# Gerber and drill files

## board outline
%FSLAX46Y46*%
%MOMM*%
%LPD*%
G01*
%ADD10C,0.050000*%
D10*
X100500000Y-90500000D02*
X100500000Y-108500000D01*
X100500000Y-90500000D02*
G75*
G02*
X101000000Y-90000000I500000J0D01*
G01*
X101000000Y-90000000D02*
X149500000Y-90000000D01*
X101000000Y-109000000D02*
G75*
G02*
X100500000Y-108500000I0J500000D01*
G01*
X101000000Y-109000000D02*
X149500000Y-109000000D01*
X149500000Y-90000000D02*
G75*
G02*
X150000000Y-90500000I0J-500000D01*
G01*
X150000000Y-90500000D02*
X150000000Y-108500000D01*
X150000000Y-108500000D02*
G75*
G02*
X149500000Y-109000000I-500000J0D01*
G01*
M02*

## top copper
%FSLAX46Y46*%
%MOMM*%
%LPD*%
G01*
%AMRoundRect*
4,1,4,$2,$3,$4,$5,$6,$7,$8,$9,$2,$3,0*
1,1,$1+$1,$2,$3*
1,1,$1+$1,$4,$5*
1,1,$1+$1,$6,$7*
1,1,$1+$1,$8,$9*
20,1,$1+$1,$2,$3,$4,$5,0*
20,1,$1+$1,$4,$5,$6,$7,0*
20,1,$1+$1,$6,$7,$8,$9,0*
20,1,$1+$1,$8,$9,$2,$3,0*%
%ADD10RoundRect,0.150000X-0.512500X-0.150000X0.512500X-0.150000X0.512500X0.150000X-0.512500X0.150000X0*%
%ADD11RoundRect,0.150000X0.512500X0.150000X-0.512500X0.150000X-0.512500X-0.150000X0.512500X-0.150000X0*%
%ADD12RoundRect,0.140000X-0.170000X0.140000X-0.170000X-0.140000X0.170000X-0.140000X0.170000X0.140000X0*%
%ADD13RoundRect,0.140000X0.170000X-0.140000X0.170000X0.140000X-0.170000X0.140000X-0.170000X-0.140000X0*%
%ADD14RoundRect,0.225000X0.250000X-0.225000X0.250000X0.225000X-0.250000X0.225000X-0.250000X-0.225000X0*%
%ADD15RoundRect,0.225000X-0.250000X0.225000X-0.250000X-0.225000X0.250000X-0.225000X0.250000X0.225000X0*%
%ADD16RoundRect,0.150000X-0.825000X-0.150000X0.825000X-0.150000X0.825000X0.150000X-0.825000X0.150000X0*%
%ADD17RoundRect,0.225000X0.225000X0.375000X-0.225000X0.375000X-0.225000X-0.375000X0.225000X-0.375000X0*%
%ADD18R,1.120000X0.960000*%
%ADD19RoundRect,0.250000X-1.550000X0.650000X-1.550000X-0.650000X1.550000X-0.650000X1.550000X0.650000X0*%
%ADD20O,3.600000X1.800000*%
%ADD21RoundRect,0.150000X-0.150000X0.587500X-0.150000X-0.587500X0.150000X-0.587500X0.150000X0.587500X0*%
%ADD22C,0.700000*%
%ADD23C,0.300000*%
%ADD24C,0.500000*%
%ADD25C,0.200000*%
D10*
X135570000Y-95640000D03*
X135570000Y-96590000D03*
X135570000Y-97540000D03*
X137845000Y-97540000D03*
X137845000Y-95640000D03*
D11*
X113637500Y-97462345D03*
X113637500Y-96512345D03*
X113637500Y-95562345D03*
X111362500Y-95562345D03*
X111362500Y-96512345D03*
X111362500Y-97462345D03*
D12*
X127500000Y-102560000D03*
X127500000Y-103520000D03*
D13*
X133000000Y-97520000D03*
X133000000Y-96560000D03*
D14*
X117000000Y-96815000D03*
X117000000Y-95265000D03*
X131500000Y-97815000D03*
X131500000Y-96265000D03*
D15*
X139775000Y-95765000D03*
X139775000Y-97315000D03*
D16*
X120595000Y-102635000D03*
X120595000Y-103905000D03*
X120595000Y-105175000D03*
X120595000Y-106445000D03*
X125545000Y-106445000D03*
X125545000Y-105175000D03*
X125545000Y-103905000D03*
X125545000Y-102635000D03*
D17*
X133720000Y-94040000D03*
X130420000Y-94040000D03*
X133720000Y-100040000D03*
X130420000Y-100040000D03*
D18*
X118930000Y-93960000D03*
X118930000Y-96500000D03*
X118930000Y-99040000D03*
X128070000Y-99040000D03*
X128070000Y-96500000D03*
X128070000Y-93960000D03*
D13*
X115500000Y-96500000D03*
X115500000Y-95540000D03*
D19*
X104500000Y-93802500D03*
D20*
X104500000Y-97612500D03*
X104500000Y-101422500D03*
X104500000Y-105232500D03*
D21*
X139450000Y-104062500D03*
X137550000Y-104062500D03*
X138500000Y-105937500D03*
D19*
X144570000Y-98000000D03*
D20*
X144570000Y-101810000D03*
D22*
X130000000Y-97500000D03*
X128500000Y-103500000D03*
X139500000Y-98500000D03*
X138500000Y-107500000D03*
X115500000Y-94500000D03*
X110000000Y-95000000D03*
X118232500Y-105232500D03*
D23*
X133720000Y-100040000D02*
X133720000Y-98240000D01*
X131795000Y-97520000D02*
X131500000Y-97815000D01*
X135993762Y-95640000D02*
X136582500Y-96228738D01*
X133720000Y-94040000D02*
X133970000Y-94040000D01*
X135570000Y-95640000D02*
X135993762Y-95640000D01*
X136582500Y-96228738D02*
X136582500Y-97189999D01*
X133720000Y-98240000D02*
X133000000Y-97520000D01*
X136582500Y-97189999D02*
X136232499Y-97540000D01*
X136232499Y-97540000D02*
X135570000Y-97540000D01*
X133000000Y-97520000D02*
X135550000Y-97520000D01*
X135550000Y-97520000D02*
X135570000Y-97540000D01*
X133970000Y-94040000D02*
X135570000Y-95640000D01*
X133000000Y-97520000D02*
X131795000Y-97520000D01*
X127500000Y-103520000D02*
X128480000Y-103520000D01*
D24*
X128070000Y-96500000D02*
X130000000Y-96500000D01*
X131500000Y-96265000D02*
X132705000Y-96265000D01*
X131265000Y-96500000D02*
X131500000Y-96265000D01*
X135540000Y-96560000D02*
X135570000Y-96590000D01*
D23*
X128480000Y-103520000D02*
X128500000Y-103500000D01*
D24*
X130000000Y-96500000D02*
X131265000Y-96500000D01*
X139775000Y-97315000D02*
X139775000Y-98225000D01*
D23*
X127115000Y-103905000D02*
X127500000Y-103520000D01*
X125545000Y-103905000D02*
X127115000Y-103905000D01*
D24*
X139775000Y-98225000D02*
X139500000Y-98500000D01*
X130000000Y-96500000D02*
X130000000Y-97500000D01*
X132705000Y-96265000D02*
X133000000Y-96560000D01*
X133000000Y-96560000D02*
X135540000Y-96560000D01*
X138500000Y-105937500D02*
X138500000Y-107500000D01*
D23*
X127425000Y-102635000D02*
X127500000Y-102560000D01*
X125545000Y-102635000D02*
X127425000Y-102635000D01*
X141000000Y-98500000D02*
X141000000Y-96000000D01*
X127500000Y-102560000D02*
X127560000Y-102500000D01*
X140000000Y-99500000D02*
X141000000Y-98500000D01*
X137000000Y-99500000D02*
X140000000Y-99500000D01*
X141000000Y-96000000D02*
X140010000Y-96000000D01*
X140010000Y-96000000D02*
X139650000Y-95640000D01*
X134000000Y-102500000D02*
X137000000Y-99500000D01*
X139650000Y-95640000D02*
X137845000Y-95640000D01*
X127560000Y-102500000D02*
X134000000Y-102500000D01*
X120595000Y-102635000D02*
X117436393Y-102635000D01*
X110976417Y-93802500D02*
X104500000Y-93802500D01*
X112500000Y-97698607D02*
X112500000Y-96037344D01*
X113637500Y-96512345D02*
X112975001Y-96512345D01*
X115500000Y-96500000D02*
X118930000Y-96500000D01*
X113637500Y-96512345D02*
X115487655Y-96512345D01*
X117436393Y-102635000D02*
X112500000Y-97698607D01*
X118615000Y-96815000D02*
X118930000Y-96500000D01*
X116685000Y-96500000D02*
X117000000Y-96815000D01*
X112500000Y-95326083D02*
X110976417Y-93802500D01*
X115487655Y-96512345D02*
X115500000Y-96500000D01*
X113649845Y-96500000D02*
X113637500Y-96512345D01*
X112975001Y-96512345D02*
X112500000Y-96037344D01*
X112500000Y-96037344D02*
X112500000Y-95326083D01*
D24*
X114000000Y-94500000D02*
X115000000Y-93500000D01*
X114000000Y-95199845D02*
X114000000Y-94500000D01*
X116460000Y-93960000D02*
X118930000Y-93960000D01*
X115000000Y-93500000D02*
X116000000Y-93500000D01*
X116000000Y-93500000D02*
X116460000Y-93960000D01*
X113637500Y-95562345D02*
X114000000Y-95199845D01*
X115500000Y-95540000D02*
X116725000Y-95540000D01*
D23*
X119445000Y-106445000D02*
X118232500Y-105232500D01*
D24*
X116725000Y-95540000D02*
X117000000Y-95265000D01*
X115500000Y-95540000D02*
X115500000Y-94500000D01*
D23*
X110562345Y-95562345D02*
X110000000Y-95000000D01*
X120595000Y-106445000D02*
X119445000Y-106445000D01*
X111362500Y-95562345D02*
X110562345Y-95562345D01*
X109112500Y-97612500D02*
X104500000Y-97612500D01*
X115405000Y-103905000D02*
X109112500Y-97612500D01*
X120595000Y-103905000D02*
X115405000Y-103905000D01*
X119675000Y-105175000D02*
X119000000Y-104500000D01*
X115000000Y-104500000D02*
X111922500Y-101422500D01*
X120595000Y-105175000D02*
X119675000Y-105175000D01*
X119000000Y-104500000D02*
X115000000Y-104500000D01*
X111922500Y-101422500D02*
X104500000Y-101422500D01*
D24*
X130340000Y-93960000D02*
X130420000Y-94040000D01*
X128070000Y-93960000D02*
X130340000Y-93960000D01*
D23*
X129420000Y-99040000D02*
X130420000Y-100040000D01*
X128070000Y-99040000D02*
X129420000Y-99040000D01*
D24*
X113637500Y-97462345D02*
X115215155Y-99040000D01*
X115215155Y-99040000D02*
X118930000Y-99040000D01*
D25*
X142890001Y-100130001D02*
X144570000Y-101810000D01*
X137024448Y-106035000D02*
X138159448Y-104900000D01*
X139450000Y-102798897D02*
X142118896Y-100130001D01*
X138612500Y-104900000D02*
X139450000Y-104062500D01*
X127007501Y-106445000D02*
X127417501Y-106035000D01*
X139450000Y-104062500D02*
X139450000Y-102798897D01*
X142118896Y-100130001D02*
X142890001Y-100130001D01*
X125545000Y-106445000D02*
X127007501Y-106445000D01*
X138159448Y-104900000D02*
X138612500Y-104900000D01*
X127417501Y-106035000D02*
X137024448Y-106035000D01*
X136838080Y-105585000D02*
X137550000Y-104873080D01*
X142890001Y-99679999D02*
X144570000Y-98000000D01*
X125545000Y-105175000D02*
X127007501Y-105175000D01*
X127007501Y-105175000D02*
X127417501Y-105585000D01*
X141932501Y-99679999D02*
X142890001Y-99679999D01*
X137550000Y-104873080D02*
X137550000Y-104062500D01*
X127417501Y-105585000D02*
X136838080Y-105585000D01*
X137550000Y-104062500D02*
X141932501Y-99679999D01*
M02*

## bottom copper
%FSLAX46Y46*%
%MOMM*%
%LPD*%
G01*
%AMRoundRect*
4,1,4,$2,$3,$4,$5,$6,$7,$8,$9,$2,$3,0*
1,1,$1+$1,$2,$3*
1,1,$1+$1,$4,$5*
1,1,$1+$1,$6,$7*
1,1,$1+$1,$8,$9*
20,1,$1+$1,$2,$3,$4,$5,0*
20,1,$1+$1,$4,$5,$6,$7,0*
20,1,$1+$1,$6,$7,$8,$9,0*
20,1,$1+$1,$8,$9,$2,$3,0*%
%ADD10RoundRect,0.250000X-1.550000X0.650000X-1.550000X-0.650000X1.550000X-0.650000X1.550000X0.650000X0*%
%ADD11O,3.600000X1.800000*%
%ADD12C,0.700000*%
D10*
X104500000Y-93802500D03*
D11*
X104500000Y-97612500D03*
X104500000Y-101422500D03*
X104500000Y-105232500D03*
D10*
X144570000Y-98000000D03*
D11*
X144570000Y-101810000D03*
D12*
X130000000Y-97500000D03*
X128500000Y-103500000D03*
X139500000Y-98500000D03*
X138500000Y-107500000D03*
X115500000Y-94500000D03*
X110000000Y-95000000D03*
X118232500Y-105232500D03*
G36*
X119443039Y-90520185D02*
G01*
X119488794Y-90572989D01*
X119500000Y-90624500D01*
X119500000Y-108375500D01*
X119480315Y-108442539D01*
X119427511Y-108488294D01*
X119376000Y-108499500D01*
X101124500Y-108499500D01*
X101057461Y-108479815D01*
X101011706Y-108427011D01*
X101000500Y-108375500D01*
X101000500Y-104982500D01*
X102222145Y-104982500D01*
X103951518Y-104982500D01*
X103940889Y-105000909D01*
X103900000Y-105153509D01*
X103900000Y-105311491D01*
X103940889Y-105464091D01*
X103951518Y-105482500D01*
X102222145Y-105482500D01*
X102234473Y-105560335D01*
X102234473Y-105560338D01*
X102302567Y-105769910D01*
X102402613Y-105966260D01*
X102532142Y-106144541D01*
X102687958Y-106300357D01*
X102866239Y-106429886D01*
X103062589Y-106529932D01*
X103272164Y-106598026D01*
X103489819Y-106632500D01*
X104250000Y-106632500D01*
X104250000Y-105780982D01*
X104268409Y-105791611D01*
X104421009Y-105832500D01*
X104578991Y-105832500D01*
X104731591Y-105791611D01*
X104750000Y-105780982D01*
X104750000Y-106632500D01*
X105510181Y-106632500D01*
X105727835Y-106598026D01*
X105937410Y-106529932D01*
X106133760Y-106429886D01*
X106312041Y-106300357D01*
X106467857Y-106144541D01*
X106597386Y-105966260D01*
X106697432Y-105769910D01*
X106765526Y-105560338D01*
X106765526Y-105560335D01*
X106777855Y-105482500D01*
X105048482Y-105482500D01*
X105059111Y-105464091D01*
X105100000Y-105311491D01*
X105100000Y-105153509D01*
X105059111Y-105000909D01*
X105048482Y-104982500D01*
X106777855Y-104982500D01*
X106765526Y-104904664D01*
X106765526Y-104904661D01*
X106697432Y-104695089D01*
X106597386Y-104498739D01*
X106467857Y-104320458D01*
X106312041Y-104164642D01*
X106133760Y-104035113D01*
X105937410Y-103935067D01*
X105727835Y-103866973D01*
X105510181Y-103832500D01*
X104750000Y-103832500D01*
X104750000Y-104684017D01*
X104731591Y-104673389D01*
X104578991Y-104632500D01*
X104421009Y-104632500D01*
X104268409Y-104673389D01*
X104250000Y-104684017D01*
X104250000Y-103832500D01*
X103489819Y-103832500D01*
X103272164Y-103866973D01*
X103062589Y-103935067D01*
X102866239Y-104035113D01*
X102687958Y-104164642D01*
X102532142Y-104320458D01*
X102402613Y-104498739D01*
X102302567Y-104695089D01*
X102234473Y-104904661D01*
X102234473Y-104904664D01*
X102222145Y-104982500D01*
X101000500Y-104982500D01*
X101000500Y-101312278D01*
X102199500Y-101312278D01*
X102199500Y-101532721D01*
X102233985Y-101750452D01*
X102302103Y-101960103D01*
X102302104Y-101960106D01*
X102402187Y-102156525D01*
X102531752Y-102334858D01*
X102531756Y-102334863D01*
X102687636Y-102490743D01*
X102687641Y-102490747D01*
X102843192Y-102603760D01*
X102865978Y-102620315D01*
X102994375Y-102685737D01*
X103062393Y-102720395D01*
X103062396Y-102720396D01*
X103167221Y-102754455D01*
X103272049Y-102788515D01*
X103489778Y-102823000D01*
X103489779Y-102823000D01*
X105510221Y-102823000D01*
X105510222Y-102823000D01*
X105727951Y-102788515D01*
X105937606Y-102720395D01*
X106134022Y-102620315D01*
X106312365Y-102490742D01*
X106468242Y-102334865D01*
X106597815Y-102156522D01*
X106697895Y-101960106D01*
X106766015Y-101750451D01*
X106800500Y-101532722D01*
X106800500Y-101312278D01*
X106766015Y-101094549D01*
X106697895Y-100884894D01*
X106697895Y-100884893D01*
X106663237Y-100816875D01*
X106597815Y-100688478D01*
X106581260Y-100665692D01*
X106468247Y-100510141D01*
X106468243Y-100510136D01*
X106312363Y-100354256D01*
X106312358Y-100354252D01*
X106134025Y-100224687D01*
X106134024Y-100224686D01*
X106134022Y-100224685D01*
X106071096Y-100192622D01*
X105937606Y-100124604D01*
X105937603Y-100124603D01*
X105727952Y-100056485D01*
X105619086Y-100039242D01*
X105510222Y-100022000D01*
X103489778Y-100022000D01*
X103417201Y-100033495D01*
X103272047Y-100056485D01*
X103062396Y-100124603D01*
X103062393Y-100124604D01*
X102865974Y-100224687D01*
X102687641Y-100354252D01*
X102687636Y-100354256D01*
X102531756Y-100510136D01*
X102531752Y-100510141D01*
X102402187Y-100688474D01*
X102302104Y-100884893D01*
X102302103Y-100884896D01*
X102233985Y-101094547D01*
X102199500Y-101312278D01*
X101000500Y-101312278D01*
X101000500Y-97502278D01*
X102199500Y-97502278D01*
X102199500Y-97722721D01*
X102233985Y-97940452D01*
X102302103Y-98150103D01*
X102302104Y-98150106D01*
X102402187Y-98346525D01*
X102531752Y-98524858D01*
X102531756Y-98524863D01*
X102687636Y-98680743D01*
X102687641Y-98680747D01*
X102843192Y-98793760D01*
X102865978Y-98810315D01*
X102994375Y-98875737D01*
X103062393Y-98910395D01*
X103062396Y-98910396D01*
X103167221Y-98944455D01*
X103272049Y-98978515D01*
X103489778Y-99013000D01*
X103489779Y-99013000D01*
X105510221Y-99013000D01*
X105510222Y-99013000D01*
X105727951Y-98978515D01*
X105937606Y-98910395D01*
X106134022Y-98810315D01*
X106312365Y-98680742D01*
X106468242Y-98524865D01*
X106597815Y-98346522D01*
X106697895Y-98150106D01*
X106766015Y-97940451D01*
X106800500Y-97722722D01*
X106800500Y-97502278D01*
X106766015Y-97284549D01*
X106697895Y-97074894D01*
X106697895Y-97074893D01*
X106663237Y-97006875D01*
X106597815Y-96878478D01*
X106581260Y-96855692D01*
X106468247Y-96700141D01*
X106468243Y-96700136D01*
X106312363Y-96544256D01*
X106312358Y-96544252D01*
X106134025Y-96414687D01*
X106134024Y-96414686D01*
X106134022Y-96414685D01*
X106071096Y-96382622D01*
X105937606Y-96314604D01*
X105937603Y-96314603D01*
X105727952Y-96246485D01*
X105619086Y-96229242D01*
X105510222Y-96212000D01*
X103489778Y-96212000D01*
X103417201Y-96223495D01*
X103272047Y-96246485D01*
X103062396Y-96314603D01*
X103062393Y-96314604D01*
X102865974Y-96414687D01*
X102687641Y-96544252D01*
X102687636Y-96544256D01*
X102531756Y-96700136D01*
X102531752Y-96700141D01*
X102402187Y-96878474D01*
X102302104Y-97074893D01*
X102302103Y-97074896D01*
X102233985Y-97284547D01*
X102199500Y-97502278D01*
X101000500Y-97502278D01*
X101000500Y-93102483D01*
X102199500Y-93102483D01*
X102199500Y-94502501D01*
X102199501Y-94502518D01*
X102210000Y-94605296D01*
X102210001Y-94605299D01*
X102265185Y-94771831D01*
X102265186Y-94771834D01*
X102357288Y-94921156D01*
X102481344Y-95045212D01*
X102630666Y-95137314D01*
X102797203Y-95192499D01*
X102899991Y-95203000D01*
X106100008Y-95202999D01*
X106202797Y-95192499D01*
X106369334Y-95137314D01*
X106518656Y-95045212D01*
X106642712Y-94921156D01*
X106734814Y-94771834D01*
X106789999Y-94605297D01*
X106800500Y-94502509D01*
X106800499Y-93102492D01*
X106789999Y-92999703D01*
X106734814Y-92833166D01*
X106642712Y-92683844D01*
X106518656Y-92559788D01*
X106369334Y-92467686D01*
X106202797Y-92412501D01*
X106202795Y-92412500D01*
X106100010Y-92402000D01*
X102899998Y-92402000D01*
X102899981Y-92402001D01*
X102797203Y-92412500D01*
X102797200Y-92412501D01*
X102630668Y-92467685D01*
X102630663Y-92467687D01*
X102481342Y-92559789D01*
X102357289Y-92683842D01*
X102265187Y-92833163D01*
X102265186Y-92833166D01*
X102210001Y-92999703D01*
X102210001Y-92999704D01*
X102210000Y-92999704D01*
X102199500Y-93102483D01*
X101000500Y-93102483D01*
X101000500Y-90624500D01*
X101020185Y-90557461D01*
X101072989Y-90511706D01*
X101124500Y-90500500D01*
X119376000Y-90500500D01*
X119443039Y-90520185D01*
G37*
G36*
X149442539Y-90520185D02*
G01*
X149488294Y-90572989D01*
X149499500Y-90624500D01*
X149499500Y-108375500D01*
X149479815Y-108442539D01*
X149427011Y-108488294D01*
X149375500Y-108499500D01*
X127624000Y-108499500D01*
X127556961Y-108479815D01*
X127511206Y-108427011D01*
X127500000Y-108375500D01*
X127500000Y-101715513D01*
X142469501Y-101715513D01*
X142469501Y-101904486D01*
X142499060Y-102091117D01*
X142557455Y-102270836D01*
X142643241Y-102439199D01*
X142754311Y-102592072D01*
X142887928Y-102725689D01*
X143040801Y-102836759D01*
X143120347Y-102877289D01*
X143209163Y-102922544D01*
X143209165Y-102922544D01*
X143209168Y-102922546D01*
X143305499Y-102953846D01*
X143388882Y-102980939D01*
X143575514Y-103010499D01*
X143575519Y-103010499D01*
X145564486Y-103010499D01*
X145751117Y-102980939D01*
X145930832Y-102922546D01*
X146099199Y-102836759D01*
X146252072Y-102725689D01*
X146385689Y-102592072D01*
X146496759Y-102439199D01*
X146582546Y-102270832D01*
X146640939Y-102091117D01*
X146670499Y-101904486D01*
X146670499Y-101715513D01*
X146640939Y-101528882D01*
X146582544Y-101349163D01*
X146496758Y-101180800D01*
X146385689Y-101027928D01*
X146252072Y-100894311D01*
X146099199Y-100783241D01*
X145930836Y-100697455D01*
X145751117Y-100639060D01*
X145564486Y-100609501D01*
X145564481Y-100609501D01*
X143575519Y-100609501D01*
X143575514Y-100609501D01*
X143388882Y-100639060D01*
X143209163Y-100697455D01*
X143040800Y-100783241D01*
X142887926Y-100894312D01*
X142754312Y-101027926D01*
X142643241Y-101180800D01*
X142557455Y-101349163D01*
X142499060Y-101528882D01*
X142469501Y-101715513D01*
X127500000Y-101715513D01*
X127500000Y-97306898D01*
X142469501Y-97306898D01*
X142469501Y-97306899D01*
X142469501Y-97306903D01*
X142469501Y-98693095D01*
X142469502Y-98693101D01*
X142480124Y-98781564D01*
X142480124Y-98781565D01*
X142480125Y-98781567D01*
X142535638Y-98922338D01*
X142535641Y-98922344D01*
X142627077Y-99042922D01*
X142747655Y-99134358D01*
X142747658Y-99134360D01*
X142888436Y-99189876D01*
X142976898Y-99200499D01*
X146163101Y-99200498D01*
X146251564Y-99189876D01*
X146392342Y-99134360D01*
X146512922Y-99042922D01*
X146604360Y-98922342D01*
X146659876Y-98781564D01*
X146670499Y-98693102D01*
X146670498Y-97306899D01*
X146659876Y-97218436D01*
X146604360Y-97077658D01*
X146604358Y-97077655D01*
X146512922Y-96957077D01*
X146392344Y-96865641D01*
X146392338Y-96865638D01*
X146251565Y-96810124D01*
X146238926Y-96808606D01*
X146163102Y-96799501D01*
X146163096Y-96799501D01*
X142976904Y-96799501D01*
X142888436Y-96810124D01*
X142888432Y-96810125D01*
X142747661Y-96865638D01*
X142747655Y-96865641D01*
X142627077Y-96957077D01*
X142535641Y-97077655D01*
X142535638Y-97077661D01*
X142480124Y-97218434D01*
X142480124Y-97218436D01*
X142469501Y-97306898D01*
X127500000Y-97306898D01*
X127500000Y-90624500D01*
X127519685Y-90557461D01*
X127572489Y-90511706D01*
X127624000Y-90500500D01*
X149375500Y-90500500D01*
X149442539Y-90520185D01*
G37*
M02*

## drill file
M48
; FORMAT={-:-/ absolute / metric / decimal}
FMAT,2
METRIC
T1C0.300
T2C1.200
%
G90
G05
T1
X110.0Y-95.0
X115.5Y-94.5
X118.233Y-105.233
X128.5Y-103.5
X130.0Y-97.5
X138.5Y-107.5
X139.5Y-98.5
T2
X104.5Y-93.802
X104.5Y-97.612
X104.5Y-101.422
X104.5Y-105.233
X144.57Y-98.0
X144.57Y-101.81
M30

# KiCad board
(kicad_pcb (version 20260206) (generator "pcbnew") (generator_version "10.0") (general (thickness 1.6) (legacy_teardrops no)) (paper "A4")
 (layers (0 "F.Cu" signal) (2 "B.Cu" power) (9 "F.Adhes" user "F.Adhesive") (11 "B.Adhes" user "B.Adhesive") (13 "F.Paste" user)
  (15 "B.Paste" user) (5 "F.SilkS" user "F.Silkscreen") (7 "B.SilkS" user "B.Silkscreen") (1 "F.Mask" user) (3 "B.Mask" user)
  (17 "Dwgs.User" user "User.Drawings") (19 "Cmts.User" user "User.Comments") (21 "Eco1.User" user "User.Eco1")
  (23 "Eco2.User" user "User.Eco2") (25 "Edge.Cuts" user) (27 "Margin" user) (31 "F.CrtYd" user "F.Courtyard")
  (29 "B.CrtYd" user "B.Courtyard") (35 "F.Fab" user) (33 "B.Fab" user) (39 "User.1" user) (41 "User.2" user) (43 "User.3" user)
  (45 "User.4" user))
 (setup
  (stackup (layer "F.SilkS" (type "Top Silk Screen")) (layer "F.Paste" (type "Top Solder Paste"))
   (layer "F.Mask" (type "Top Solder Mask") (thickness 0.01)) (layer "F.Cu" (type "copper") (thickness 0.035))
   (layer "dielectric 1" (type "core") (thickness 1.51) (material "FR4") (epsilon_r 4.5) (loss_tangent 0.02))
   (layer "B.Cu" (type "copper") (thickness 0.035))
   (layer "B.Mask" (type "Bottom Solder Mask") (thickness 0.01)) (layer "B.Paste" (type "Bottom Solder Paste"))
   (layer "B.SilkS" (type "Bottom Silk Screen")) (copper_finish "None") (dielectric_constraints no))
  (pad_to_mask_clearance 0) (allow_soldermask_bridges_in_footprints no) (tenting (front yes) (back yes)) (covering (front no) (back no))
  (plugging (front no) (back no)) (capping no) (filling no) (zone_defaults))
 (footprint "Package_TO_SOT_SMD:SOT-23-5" (layer "F.Cu") (at 136.7075 96.59)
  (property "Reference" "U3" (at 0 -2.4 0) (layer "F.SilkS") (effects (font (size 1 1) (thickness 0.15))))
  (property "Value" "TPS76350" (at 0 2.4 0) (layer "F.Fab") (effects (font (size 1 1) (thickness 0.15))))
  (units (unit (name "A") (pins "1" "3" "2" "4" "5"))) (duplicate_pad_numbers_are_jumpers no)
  (pad "1" smd roundrect (at -1.1375 -0.95) (size 1.325 0.6) (layers "F.Cu" "F.Mask" "F.Paste") (roundrect_rratio 0.25) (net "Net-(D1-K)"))
  (pad "2" smd roundrect (at -1.1375 0) (size 1.325 0.6) (layers "F.Cu" "F.Mask" "F.Paste") (roundrect_rratio 0.25) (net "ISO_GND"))
  (pad "3" smd roundrect (at -1.1375 0.95) (size 1.325 0.6) (layers "F.Cu" "F.Mask" "F.Paste") (roundrect_rratio 0.25) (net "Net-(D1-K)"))
  (pad "4" smd roundrect (at 1.1375 0.95) (size 1.325 0.6) (layers "F.Cu" "F.Mask" "F.Paste") (roundrect_rratio 0.25)
   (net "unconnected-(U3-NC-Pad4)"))
  (pad "5" smd roundrect (at 1.1375 -0.95) (size 1.325 0.6) (layers "F.Cu" "F.Mask" "F.Paste") (roundrect_rratio 0.25) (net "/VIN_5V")))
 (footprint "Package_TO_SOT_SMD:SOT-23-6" (layer "F.Cu") (at 112.5 96.512345 180)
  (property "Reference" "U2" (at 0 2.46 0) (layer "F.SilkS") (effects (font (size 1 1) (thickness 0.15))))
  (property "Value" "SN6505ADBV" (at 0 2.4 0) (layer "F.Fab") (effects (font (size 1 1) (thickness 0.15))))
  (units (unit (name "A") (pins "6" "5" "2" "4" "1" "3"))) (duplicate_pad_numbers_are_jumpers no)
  (pad "1" smd roundrect (at -1.1375 -0.95 180) (size 1.325 0.6) (layers "F.Cu" "F.Mask" "F.Paste") (roundrect_rratio 0.25)
   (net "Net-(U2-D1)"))
  (pad "2" smd roundrect (at -1.1375 0 180) (size 1.325 0.6) (layers "F.Cu" "F.Mask" "F.Paste") (roundrect_rratio 0.25) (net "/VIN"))
  (pad "3" smd roundrect (at -1.1375 0.95 180) (size 1.325 0.6) (layers "F.Cu" "F.Mask" "F.Paste") (roundrect_rratio 0.25)
   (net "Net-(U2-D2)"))
  (pad "4" smd roundrect (at 1.1375 0.95 180) (size 1.325 0.6) (layers "F.Cu" "F.Mask" "F.Paste") (roundrect_rratio 0.25) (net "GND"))
  (pad "5" smd roundrect (at 1.1375 0 180) (size 1.325 0.6) (layers "F.Cu" "F.Mask" "F.Paste") (roundrect_rratio 0.25)
   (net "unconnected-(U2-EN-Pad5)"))
  (pad "6" smd roundrect (at 1.1375 -0.95 180) (size 1.325 0.6) (layers "F.Cu" "F.Mask" "F.Paste") (roundrect_rratio 0.25)
   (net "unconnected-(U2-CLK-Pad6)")))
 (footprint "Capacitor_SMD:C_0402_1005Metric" (layer "F.Cu") (at 127.5 103.04 -90)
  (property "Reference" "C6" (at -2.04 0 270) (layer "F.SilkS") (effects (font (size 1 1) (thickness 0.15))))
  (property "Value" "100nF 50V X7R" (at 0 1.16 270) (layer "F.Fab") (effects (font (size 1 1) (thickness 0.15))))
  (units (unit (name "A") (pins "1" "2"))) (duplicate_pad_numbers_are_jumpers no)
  (pad "1" smd roundrect (at -0.48 0 270) (size 0.56 0.62) (layers "F.Cu" "F.Mask" "F.Paste") (roundrect_rratio 0.25) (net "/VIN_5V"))
  (pad "2" smd roundrect (at 0.48 0 270) (size 0.56 0.62) (layers "F.Cu" "F.Mask" "F.Paste") (roundrect_rratio 0.25) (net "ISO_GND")))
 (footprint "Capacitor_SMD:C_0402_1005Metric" (layer "F.Cu") (at 133 97.04 90)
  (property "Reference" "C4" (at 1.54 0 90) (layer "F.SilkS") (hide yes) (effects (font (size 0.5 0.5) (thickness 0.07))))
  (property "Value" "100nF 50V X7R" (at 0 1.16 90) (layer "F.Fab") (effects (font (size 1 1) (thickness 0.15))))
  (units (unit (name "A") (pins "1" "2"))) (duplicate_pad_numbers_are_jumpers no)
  (pad "1" smd roundrect (at -0.48 0 90) (size 0.56 0.62) (layers "F.Cu" "F.Mask" "F.Paste") (roundrect_rratio 0.25) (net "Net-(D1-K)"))
  (pad "2" smd roundrect (at 0.48 0 90) (size 0.56 0.62) (layers "F.Cu" "F.Mask" "F.Paste") (roundrect_rratio 0.25) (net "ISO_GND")))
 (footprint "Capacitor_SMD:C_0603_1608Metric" (layer "F.Cu") (at 117 96.04 90)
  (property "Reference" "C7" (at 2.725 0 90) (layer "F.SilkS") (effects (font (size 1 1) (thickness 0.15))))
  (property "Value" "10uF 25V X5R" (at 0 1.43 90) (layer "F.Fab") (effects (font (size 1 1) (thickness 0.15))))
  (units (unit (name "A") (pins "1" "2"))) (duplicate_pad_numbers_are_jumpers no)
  (pad "1" smd roundrect (at -0.775 0 90) (size 0.9 0.95) (layers "F.Cu" "F.Mask" "F.Paste") (roundrect_rratio 0.25) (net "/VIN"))
  (pad "2" smd roundrect (at 0.775 0 90) (size 0.9 0.95) (layers "F.Cu" "F.Mask" "F.Paste") (roundrect_rratio 0.25) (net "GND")))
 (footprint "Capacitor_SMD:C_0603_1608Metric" (layer "F.Cu") (at 131.5 97.04 90)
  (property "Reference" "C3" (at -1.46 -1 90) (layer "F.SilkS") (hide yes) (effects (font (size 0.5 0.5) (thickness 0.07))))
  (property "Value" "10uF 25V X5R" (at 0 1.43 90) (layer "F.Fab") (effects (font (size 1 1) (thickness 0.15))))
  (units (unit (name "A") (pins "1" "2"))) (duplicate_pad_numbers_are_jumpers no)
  (pad "1" smd roundrect (at -0.775 0 90) (size 0.9 0.95) (layers "F.Cu" "F.Mask" "F.Paste") (roundrect_rratio 0.25) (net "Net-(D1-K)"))
  (pad "2" smd roundrect (at 0.775 0 90) (size 0.9 0.95) (layers "F.Cu" "F.Mask" "F.Paste") (roundrect_rratio 0.25) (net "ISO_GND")))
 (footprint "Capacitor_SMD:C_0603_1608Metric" (layer "F.Cu") (at 139.775 96.54 -90)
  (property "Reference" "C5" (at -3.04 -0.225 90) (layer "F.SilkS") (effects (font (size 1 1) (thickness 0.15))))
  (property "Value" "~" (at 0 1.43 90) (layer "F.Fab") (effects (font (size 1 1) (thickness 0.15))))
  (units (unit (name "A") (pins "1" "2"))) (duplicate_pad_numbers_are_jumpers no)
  (pad "1" smd roundrect (at -0.775 0 270) (size 0.9 0.95) (layers "F.Cu" "F.Mask" "F.Paste") (roundrect_rratio 0.25) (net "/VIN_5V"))
  (pad "2" smd roundrect (at 0.775 0 270) (size 0.9 0.95) (layers "F.Cu" "F.Mask" "F.Paste") (roundrect_rratio 0.25) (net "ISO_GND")))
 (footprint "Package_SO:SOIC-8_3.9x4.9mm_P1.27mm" (layer "F.Cu") (at 123.07 104.54)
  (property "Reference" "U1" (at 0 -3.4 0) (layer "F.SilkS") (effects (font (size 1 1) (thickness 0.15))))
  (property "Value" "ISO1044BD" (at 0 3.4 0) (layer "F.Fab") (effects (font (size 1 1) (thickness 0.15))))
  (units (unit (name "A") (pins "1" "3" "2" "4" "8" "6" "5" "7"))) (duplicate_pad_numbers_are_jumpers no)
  (pad "1" smd roundrect (at -2.475 -1.905) (size 1.95 0.6) (layers "F.Cu" "F.Mask" "F.Paste") (roundrect_rratio 0.25) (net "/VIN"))
  (pad "2" smd roundrect (at -2.475 -0.635) (size 1.95 0.6) (layers "F.Cu" "F.Mask" "F.Paste") (roundrect_rratio 0.25) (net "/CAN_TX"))
  (pad "3" smd roundrect (at -2.475 0.635) (size 1.95 0.6) (layers "F.Cu" "F.Mask" "F.Paste") (roundrect_rratio 0.25) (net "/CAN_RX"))
  (pad "4" smd roundrect (at -2.475 1.905) (size 1.95 0.6) (layers "F.Cu" "F.Mask" "F.Paste") (roundrect_rratio 0.25) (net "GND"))
  (pad "5" smd roundrect (at 2.475 1.905) (size 1.95 0.6) (layers "F.Cu" "F.Mask" "F.Paste") (roundrect_rratio 0.25) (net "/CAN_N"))
  (pad "6" smd roundrect (at 2.475 0.635) (size 1.95 0.6) (layers "F.Cu" "F.Mask" "F.Paste") (roundrect_rratio 0.25) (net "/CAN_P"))
  (pad "7" smd roundrect (at 2.475 -0.635) (size 1.95 0.6) (layers "F.Cu" "F.Mask" "F.Paste") (roundrect_rratio 0.25) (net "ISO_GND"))
  (pad "8" smd roundrect (at 2.475 -1.905) (size 1.95 0.6) (layers "F.Cu" "F.Mask" "F.Paste") (roundrect_rratio 0.25) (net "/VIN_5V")))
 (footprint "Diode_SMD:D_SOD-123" (layer "F.Cu") (at 132.07 94.04 180)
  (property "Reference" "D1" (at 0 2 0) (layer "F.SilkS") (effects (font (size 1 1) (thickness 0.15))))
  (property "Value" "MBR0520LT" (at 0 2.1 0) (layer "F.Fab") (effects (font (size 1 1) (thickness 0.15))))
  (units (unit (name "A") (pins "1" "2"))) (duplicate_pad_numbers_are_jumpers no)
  (pad "1" smd roundrect (at -1.65 0 180) (size 0.9 1.2) (layers "F.Cu" "F.Mask" "F.Paste") (roundrect_rratio 0.25) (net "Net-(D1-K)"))
  (pad "2" smd roundrect (at 1.65 0 180) (size 0.9 1.2) (layers "F.Cu" "F.Mask" "F.Paste") (roundrect_rratio 0.25) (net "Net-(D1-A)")))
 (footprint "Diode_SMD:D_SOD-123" (layer "F.Cu") (at 132.07 100.04 180)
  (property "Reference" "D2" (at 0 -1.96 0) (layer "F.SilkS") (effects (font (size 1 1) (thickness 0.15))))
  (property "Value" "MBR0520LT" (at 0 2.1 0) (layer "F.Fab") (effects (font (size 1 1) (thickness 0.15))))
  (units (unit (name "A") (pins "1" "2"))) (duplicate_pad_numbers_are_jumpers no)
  (pad "1" smd roundrect (at -1.65 0 180) (size 0.9 1.2) (layers "F.Cu" "F.Mask" "F.Paste") (roundrect_rratio 0.25) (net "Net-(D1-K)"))
  (pad "2" smd roundrect (at 1.65 0 180) (size 0.9 1.2) (layers "F.Cu" "F.Mask" "F.Paste") (roundrect_rratio 0.25) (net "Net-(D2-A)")))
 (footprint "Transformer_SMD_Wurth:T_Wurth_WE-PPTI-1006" (layer "F.Cu") (at 123.5 96.5)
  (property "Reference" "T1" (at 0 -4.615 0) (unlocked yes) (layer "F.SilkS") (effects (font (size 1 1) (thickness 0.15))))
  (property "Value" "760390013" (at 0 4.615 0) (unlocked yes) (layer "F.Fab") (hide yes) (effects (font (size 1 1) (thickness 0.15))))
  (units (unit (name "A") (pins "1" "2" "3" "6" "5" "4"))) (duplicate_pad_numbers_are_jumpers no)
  (pad "1" smd rect (at -4.57 -2.54) (size 1.12 0.96) (layers "F.Cu" "F.Mask" "F.Paste") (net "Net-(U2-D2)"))
  (pad "2" smd rect (at -4.57 0) (size 1.12 0.96) (layers "F.Cu" "F.Mask" "F.Paste") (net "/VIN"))
  (pad "3" smd rect (at -4.57 2.54) (size 1.12 0.96) (layers "F.Cu" "F.Mask" "F.Paste") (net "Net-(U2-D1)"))
  (pad "4" smd rect (at 4.57 2.54) (size 1.12 0.96) (layers "F.Cu" "F.Mask" "F.Paste") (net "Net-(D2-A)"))
  (pad "5" smd rect (at 4.57 0) (size 1.12 0.96) (layers "F.Cu" "F.Mask" "F.Paste") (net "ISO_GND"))
  (pad "6" smd rect (at 4.57 -2.54) (size 1.12 0.96) (layers "F.Cu" "F.Mask" "F.Paste") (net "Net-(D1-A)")))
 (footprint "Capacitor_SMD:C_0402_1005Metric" (layer "F.Cu") (at 115.5 96.02 90)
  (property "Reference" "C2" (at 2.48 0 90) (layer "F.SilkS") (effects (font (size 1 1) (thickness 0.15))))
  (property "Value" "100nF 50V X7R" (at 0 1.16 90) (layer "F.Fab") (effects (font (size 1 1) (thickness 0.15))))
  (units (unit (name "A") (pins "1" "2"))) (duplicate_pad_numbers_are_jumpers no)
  (pad "1" smd roundrect (at -0.48 0 90) (size 0.56 0.62) (layers "F.Cu" "F.Mask" "F.Paste") (roundrect_rratio 0.25) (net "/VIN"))
  (pad "2" smd roundrect (at 0.48 0 90) (size 0.56 0.62) (layers "F.Cu" "F.Mask" "F.Paste") (roundrect_rratio 0.25) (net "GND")))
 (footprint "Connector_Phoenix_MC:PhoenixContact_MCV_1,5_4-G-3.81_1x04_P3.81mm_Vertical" (layer "F.Cu") (at 104.5 93.8025 -90)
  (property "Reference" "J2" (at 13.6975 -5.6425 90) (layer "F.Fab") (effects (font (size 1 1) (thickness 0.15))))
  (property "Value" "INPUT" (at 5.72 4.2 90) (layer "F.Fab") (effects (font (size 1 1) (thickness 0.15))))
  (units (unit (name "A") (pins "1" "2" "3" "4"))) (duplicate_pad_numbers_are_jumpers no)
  (pad "1" thru_hole roundrect (at 0 0 270) (size 1.8 3.6) (drill 1.2) (layers "*.Cu" "*.Mask") (remove_unused_layers no)
   (roundrect_rratio 0.138889) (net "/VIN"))
  (pad "2" thru_hole oval (at 3.81 0 270) (size 1.8 3.6) (drill 1.2) (layers "*.Cu" "*.Mask") (remove_unused_layers no) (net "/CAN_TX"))
  (pad "3" thru_hole oval (at 7.62 0 270) (size 1.8 3.6) (drill 1.2) (layers "*.Cu" "*.Mask") (remove_unused_layers no) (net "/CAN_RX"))
  (pad "4" thru_hole oval (at 11.43 0 270) (size 1.8 3.6) (drill 1.2) (layers "*.Cu" "*.Mask") (remove_unused_layers no) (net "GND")))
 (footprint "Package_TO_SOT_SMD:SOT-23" (layer "F.Cu") (at 138.5 105 -90)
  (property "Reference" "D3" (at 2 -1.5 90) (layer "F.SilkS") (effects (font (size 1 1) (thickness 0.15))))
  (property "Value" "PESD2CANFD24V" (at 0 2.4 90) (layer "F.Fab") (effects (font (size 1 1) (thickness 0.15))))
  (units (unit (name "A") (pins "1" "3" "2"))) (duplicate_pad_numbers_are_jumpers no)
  (pad "1" smd roundrect (at -0.9375 -0.95 270) (size 1.475 0.6) (layers "F.Cu" "F.Mask" "F.Paste") (roundrect_rratio 0.25) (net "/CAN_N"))
  (pad "2" smd roundrect (at -0.9375 0.95 270) (size 1.475 0.6) (layers "F.Cu" "F.Mask" "F.Paste") (roundrect_rratio 0.25) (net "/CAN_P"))
  (pad "3" smd roundrect (at 0.9375 0 270) (size 1.475 0.6) (layers "F.Cu" "F.Mask" "F.Paste") (roundrect_rratio 0.25) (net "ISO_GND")))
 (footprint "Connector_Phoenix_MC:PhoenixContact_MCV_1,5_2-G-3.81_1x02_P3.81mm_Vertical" (layer "F.Cu") (at 144.57 98 -90)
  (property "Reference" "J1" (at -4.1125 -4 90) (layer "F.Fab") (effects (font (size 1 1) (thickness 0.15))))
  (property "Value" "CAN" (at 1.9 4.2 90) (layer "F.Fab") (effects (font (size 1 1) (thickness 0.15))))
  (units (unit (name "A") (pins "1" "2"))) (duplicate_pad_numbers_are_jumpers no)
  (pad "1" thru_hole roundrect (at 0 0 270) (size 1.8 3.6) (drill 1.2) (layers "*.Cu" "*.Mask") (remove_unused_layers no)
   (roundrect_rratio 0.138889) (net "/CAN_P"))
  (pad "2" thru_hole oval (at 3.81 0 270) (size 1.8 3.6) (drill 1.2) (layers "*.Cu" "*.Mask") (remove_unused_layers no) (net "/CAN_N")))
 (gr_line (start 100.5 90.5) (end 100.5 108.5) (stroke (width 0.05) (type default)) (layer "Edge.Cuts"))
 (gr_arc (start 100.5 90.5) (mid 100.646447 90.146447) (end 101 90) (stroke (width 0.05) (type default)) (layer "Edge.Cuts"))
 (gr_line (start 101 90) (end 149.5 90) (stroke (width 0.05) (type default)) (layer "Edge.Cuts"))
 (gr_arc (start 101 109) (mid 100.646447 108.853553) (end 100.5 108.5) (stroke (width 0.05) (type default)) (layer "Edge.Cuts"))
 (gr_line (start 101 109) (end 149.5 109) (stroke (width 0.05) (type default)) (layer "Edge.Cuts"))
 (gr_arc (start 149.5 90) (mid 149.853553 90.146447) (end 150 90.5) (stroke (width 0.05) (type default)) (layer "Edge.Cuts"))
 (gr_line (start 150 90.5) (end 150 108.5) (stroke (width 0.05) (type default)) (layer "Edge.Cuts"))
 (gr_arc (start 150 108.5) (mid 149.853553 108.853553) (end 149.5 109) (stroke (width 0.05) (type default)) (layer "Edge.Cuts"))
 (segment (start 133.72 100.04) (end 133.72 98.24) (width 0.3) (layer "F.Cu") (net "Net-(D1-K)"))
 (segment (start 131.795 97.52) (end 131.5 97.815) (width 0.3) (layer "F.Cu") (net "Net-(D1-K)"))
 (segment (start 135.993762 95.64) (end 136.5825 96.228738) (width 0.3) (layer "F.Cu") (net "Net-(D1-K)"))
 (segment (start 133.72 94.04) (end 133.97 94.04) (width 0.3) (layer "F.Cu") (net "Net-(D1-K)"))
 (segment (start 135.57 95.64) (end 135.993762 95.64) (width 0.3) (layer "F.Cu") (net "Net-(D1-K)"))
 (segment (start 136.5825 96.228738) (end 136.5825 97.189999) (width 0.3) (layer "F.Cu") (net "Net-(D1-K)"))
 (segment (start 133.72 98.24) (end 133 97.52) (width 0.3) (layer "F.Cu") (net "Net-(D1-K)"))
 (segment (start 136.5825 97.189999) (end 136.232499 97.54) (width 0.3) (layer "F.Cu") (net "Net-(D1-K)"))
 (segment (start 136.232499 97.54) (end 135.57 97.54) (width 0.3) (layer "F.Cu") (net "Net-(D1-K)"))
 (segment (start 133 97.52) (end 135.55 97.52) (width 0.3) (layer "F.Cu") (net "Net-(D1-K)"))
 (segment (start 135.55 97.52) (end 135.57 97.54) (width 0.3) (layer "F.Cu") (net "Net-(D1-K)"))
 (segment (start 133.97 94.04) (end 135.57 95.64) (width 0.3) (layer "F.Cu") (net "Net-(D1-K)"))
 (segment (start 133 97.52) (end 131.795 97.52) (width 0.3) (layer "F.Cu") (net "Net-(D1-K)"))
 (segment (start 127.5 103.52) (end 128.48 103.52) (width 0.3) (layer "F.Cu") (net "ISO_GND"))
 (segment (start 128.07 96.5) (end 130 96.5) (width 0.5) (layer "F.Cu") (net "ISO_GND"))
 (segment (start 131.5 96.265) (end 132.705 96.265) (width 0.5) (layer "F.Cu") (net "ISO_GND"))
 (segment (start 131.265 96.5) (end 131.5 96.265) (width 0.5) (layer "F.Cu") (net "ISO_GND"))
 (segment (start 135.54 96.56) (end 135.57 96.59) (width 0.5) (layer "F.Cu") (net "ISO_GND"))
 (segment (start 128.48 103.52) (end 128.5 103.5) (width 0.3) (layer "F.Cu") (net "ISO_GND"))
 (segment (start 130 96.5) (end 131.265 96.5) (width 0.5) (layer "F.Cu") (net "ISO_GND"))
 (segment (start 139.775 97.315) (end 139.775 98.225) (width 0.5) (layer "F.Cu") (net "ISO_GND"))
 (segment (start 127.115 103.905) (end 127.5 103.52) (width 0.3) (layer "F.Cu") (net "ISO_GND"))
 (segment (start 125.545 103.905) (end 127.115 103.905) (width 0.3) (layer "F.Cu") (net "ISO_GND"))
 (segment (start 139.775 98.225) (end 139.5 98.5) (width 0.5) (layer "F.Cu") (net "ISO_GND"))
 (segment (start 130 96.5) (end 130 97.5) (width 0.5) (layer "F.Cu") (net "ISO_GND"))
 (segment (start 132.705 96.265) (end 133 96.56) (width 0.5) (layer "F.Cu") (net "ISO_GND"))
 (segment (start 133 96.56) (end 135.54 96.56) (width 0.5) (layer "F.Cu") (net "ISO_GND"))
 (segment (start 138.5 105.9375) (end 138.5 107.5) (width 0.5) (layer "F.Cu") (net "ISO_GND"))
 (via (at 130 97.5) (size 0.7) (drill 0.3) (layers "F.Cu" "B.Cu") (free yes) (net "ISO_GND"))
 (via (at 128.5 103.5) (size 0.7) (drill 0.3) (layers "F.Cu" "B.Cu") (free yes) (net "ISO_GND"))
 (via (at 139.5 98.5) (size 0.7) (drill 0.3) (layers "F.Cu" "B.Cu") (free yes) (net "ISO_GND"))
 (via (at 138.5 107.5) (size 0.7) (drill 0.3) (layers "F.Cu" "B.Cu") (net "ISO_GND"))
 (segment (start 127.425 102.635) (end 127.5 102.56) (width 0.3) (layer "F.Cu") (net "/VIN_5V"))
 (segment (start 125.545 102.635) (end 127.425 102.635) (width 0.3) (layer "F.Cu") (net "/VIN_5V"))
 (segment (start 141 98.5) (end 141 96) (width 0.3) (layer "F.Cu") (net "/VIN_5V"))
 (segment (start 127.5 102.56) (end 127.56 102.5) (width 0.3) (layer "F.Cu") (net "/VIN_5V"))
 (segment (start 140 99.5) (end 141 98.5) (width 0.3) (layer "F.Cu") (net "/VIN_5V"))
 (segment (start 137 99.5) (end 140 99.5) (width 0.3) (layer "F.Cu") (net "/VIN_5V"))
 (segment (start 141 96) (end 140.01 96) (width 0.3) (layer "F.Cu") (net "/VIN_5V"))
 (segment (start 140.01 96) (end 139.65 95.64) (width 0.3) (layer "F.Cu") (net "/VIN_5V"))
 (segment (start 134 102.5) (end 137 99.5) (width 0.3) (layer "F.Cu") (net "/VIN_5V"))
 (segment (start 139.65 95.64) (end 137.845 95.64) (width 0.3) (layer "F.Cu") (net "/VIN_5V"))
 (segment (start 127.56 102.5) (end 134 102.5) (width 0.3) (layer "F.Cu") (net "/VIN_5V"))
 (segment (start 120.595 102.635) (end 117.436393 102.635) (width 0.3) (layer "F.Cu") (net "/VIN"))
 (segment (start 110.976417 93.8025) (end 104.5 93.8025) (width 0.3) (layer "F.Cu") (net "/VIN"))
 (segment (start 112.5 97.698607) (end 112.5 96.037344) (width 0.3) (layer "F.Cu") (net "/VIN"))
 (segment (start 113.6375 96.512345) (end 112.975001 96.512345) (width 0.3) (layer "F.Cu") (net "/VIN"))
 (segment (start 115.5 96.5) (end 118.93 96.5) (width 0.3) (layer "F.Cu") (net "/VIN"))
 (segment (start 113.6375 96.512345) (end 115.487655 96.512345) (width 0.3) (layer "F.Cu") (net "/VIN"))
 (segment (start 117.436393 102.635) (end 112.5 97.698607) (width 0.3) (layer "F.Cu") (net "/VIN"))
 (segment (start 118.615 96.815) (end 118.93 96.5) (width 0.3) (layer "F.Cu") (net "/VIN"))
 (segment (start 116.685 96.5) (end 117 96.815) (width 0.3) (layer "F.Cu") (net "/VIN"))
 (segment (start 112.5 95.326083) (end 110.976417 93.8025) (width 0.3) (layer "F.Cu") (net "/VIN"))
 (segment (start 115.487655 96.512345) (end 115.5 96.5) (width 0.3) (layer "F.Cu") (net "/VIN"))
 (segment (start 113.649845 96.5) (end 113.6375 96.512345) (width 0.3) (layer "F.Cu") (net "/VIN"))
 (segment (start 112.975001 96.512345) (end 112.5 96.037344) (width 0.3) (layer "F.Cu") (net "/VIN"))
 (segment (start 112.5 96.037344) (end 112.5 95.326083) (width 0.3) (layer "F.Cu") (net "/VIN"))
 (segment (start 114 94.5) (end 115 93.5) (width 0.5) (layer "F.Cu") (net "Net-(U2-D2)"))
 (segment (start 114 95.199845) (end 114 94.5) (width 0.5) (layer "F.Cu") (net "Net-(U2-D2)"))
 (segment (start 116.46 93.96) (end 118.93 93.96) (width 0.5) (layer "F.Cu") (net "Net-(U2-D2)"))
 (segment (start 115 93.5) (end 116 93.5) (width 0.5) (layer "F.Cu") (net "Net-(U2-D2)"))
 (segment (start 116 93.5) (end 116.46 93.96) (width 0.5) (layer "F.Cu") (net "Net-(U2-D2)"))
 (segment (start 113.6375 95.562345) (end 114 95.199845) (width 0.5) (layer "F.Cu") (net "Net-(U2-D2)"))
 (segment (start 115.5 95.54) (end 116.725 95.54) (width 0.5) (layer "F.Cu") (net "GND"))
 (segment (start 119.445 106.445) (end 118.2325 105.2325) (width 0.3) (layer "F.Cu") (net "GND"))
 (segment (start 116.725 95.54) (end 117 95.265) (width 0.5) (layer "F.Cu") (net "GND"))
 (segment (start 115.5 95.54) (end 115.5 94.5) (width 0.5) (layer "F.Cu") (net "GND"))
 (segment (start 110.562345 95.562345) (end 110 95) (width 0.3) (layer "F.Cu") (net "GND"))
 (segment (start 120.595 106.445) (end 119.445 106.445) (width 0.3) (layer "F.Cu") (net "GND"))
 (segment (start 111.3625 95.562345) (end 110.562345 95.562345) (width 0.3) (layer "F.Cu") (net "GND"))
 (via (at 115.5 94.5) (size 0.7) (drill 0.3) (layers "F.Cu" "B.Cu") (free yes) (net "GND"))
 (via (at 110 95) (size 0.7) (drill 0.3) (layers "F.Cu" "B.Cu") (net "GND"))
 (via (at 118.2325 105.2325) (size 0.7) (drill 0.3) (layers "F.Cu" "B.Cu") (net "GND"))
 (segment (start 109.1125 97.6125) (end 104.5 97.6125) (width 0.3) (layer "F.Cu") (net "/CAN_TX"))
 (segment (start 115.405 103.905) (end 109.1125 97.6125) (width 0.3) (layer "F.Cu") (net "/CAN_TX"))
 (segment (start 120.595 103.905) (end 115.405 103.905) (width 0.3) (layer "F.Cu") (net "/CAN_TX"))
 (segment (start 119.675 105.175) (end 119 104.5) (width 0.3) (layer "F.Cu") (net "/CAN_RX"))
 (segment (start 115 104.5) (end 111.9225 101.4225) (width 0.3) (layer "F.Cu") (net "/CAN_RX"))
 (segment (start 120.595 105.175) (end 119.675 105.175) (width 0.3) (layer "F.Cu") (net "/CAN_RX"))
 (segment (start 119 104.5) (end 115 104.5) (width 0.3) (layer "F.Cu") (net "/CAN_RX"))
 (segment (start 111.9225 101.4225) (end 104.5 101.4225) (width 0.3) (layer "F.Cu") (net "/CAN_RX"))
 (segment (start 130.34 93.96) (end 130.42 94.04) (width 0.5) (layer "F.Cu") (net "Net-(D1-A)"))
 (segment (start 128.07 93.96) (end 130.34 93.96) (width 0.5) (layer "F.Cu") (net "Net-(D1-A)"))
 (segment (start 129.42 99.04) (end 130.42 100.04) (width 0.3) (layer "F.Cu") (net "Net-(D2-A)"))
 (segment (start 128.07 99.04) (end 129.42 99.04) (width 0.3) (layer "F.Cu") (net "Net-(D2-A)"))
 (segment (start 113.6375 97.462345) (end 115.215155 99.04) (width 0.5) (layer "F.Cu") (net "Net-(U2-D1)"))
 (segment (start 115.215155 99.04) (end 118.93 99.04) (width 0.5) (layer "F.Cu") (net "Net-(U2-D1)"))
 (segment (start 142.890001 100.130001) (end 144.57 101.81) (width 0.2) (layer "F.Cu") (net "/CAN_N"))
 (segment (start 137.024448 106.035) (end 138.159448 104.9) (width 0.2) (layer "F.Cu") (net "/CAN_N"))
 (segment (start 139.45 102.798897) (end 142.118896 100.130001) (width 0.2) (layer "F.Cu") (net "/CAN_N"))
 (segment (start 138.6125 104.9) (end 139.45 104.0625) (width 0.2) (layer "F.Cu") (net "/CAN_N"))
 (segment (start 127.007501 106.445) (end 127.417501 106.035) (width 0.2) (layer "F.Cu") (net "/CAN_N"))
 (segment (start 139.45 104.0625) (end 139.45 102.798897) (width 0.2) (layer "F.Cu") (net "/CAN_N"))
 (segment (start 142.118896 100.130001) (end 142.890001 100.130001) (width 0.2) (layer "F.Cu") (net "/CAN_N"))
 (segment (start 125.545 106.445) (end 127.007501 106.445) (width 0.2) (layer "F.Cu") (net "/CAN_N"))
 (segment (start 138.159448 104.9) (end 138.6125 104.9) (width 0.2) (layer "F.Cu") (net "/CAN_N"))
 (segment (start 127.417501 106.035) (end 137.024448 106.035) (width 0.2) (layer "F.Cu") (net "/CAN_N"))
 (segment (start 136.83808 105.585) (end 137.55 104.87308) (width 0.2) (layer "F.Cu") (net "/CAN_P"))
 (segment (start 142.890001 99.679999) (end 144.57 98) (width 0.2) (layer "F.Cu") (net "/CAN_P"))
 (segment (start 125.545 105.175) (end 127.007501 105.175) (width 0.2) (layer "F.Cu") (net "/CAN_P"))
 (segment (start 127.007501 105.175) (end 127.417501 105.585) (width 0.2) (layer "F.Cu") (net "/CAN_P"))
 (segment (start 141.932501 99.679999) (end 142.890001 99.679999) (width 0.2) (layer "F.Cu") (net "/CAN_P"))
 (segment (start 137.55 104.87308) (end 137.55 104.0625) (width 0.2) (layer "F.Cu") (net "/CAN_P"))
 (segment (start 127.417501 105.585) (end 136.83808 105.585) (width 0.2) (layer "F.Cu") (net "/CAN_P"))
 (segment (start 137.55 104.0625) (end 141.932501 99.679999) (width 0.2) (layer "F.Cu") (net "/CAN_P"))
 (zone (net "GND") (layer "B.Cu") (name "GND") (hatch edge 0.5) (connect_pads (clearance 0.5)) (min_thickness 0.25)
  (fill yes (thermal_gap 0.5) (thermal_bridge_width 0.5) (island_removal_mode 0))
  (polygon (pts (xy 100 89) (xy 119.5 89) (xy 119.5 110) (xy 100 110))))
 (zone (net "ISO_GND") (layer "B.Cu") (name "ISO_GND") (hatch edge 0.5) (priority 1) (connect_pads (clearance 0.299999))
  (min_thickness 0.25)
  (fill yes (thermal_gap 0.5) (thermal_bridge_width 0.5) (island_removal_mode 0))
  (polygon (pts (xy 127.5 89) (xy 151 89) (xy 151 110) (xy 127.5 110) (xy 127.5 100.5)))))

